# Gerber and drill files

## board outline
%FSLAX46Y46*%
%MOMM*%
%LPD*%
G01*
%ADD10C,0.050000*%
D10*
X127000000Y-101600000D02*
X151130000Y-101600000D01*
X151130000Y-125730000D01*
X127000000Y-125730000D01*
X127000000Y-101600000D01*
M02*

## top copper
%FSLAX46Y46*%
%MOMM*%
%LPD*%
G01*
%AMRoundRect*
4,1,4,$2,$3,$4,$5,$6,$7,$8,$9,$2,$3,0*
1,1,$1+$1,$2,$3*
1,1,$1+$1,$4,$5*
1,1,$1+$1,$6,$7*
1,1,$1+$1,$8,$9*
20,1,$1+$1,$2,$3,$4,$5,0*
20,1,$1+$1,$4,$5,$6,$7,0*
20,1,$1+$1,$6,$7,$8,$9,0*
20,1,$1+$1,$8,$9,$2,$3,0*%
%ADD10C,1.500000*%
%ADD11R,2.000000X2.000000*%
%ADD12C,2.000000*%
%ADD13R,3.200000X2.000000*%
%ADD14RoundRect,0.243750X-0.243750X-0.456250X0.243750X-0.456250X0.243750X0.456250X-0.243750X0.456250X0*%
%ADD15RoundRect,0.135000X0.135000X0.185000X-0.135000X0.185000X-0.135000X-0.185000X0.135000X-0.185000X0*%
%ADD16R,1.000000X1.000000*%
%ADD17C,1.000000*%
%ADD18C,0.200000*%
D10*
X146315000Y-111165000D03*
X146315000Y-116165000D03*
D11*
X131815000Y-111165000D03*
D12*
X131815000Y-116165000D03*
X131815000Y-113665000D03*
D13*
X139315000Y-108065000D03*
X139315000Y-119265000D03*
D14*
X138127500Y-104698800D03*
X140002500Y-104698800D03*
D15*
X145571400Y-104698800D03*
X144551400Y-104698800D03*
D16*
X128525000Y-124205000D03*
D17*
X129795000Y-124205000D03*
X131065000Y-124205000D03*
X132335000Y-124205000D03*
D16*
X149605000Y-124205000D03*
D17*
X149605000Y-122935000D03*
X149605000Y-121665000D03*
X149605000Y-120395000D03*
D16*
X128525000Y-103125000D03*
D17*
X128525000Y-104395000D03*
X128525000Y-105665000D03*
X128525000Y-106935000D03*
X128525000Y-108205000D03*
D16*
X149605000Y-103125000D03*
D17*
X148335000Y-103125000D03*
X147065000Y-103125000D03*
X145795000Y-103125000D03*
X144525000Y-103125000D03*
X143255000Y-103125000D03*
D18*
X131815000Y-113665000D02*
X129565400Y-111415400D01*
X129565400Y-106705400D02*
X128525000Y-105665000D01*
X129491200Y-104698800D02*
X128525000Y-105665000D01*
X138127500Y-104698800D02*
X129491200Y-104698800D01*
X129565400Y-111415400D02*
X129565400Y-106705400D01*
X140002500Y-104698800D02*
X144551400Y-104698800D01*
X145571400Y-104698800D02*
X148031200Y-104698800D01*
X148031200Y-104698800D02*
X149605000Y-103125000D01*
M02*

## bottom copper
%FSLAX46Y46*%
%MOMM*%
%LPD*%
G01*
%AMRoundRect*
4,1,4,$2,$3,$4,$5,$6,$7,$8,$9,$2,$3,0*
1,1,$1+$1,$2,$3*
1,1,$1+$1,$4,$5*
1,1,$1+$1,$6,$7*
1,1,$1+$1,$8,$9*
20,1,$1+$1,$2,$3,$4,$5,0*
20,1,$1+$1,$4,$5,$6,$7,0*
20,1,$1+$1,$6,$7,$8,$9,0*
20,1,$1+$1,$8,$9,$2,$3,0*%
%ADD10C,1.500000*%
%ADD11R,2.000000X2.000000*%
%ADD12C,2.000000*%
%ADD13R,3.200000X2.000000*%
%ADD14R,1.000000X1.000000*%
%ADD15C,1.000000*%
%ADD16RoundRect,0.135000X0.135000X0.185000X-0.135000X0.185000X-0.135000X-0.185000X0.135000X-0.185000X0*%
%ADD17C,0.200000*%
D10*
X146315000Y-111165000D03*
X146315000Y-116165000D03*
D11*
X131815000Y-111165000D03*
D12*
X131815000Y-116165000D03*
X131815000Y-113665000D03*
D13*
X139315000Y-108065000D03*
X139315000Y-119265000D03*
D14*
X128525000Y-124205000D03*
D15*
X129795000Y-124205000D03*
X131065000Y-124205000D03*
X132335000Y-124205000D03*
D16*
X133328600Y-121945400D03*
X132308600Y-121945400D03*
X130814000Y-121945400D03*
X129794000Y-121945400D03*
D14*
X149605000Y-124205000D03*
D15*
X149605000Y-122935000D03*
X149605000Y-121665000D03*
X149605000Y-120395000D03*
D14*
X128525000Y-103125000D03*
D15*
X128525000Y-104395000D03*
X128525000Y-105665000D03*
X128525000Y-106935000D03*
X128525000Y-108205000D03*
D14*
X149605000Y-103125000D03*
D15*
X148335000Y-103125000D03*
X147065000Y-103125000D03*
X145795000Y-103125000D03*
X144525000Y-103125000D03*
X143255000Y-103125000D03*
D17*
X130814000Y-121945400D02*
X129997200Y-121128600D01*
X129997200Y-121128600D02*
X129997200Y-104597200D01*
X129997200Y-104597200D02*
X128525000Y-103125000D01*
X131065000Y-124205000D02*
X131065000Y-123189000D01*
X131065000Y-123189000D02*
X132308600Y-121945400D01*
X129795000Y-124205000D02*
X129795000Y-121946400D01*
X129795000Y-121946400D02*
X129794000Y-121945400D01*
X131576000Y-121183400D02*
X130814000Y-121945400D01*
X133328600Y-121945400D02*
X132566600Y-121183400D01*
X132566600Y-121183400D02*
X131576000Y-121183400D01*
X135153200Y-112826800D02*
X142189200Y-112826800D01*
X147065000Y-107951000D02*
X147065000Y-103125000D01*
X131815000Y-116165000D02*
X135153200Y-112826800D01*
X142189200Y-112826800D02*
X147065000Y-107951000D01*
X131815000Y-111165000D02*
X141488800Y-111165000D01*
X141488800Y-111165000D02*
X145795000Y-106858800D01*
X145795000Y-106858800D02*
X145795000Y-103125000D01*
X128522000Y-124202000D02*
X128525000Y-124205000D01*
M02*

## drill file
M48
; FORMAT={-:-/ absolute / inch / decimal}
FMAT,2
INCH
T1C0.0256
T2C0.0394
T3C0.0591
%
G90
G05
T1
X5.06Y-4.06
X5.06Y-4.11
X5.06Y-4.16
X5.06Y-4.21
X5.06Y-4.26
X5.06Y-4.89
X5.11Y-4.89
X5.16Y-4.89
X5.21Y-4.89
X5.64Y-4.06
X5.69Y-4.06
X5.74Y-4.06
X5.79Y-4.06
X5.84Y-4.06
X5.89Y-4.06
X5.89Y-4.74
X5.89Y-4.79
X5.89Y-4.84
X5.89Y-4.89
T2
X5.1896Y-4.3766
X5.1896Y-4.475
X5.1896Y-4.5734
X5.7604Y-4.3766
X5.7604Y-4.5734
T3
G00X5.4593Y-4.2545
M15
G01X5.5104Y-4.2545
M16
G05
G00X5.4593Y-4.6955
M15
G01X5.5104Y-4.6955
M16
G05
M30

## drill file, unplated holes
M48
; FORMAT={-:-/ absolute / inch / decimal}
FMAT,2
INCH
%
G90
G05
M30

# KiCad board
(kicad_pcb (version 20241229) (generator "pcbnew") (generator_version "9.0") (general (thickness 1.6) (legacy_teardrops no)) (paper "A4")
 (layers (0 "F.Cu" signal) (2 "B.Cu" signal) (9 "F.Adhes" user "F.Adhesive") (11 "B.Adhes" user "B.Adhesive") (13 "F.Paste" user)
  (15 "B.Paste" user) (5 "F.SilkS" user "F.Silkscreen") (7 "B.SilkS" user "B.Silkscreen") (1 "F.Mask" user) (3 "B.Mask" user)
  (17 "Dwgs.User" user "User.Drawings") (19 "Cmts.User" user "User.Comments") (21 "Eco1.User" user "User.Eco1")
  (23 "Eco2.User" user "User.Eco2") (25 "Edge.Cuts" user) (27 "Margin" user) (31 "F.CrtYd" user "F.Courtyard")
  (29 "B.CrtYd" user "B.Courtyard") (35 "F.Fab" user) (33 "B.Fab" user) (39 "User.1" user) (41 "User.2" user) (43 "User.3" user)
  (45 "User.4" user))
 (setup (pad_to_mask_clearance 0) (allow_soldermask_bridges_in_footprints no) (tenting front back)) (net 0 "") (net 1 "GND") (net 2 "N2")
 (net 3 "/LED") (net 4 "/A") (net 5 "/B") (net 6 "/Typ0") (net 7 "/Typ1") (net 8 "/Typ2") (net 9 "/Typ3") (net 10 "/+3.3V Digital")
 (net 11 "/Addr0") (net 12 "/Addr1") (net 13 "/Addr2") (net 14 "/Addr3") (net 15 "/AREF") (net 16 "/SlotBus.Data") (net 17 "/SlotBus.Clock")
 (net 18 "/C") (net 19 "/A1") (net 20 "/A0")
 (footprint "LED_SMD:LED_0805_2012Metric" (layer "F.Cu") (at 139.065 104.6988)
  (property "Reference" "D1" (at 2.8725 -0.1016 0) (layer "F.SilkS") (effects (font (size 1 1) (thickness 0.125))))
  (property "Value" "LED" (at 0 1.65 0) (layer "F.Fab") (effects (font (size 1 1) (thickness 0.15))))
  (pad "1" smd roundrect (at -0.9375 0) (size 0.975 1.4) (layers "F.Cu" "F.Mask" "F.Paste") (roundrect_rratio 0.25) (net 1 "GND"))
  (pad "2" smd roundrect (at 0.9375 0) (size 0.975 1.4) (layers "F.Cu" "F.Mask" "F.Paste") (roundrect_rratio 0.25) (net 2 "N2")))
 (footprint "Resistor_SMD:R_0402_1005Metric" (layer "F.Cu") (at 145.0614 104.6988 180)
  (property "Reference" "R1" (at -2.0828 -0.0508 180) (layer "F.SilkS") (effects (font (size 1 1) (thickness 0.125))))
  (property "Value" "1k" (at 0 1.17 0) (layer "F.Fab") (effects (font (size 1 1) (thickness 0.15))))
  (pad "1" smd roundrect (at -0.51 0 180) (size 0.54 0.64) (layers "F.Cu" "F.Mask" "F.Paste") (roundrect_rratio 0.25) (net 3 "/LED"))
  (pad "2" smd roundrect (at 0.51 0 180) (size 0.54 0.64) (layers "F.Cu" "F.Mask" "F.Paste") (roundrect_rratio 0.25) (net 2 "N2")))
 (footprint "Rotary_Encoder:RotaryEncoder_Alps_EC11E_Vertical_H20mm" (layer "F.Cu") (at 131.815 111.165)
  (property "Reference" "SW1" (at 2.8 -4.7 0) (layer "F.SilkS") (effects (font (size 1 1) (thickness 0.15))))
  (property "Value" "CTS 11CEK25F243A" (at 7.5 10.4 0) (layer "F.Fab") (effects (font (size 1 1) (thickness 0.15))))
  (pad "" thru_hole circle (at 14.5 0) (size 1.5 1.5) (drill 1) (layers "*.Cu" "*.Mask") (remove_unused_layers no))
  (pad "" thru_hole circle (at 14.5 5) (size 1.5 1.5) (drill 1) (layers "*.Cu" "*.Mask") (remove_unused_layers no))
  (pad "A" thru_hole rect (at 0 0) (size 2 2) (drill 1) (layers "*.Cu" "*.Mask") (remove_unused_layers no) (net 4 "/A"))
  (pad "B" thru_hole circle (at 0 5) (size 2 2) (drill 1) (layers "*.Cu" "*.Mask") (remove_unused_layers no) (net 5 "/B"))
  (pad "C" thru_hole circle (at 0 2.5) (size 2 2) (drill 1) (layers "*.Cu" "*.Mask") (remove_unused_layers no) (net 1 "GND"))
  (pad "MP" thru_hole rect (at 7.5 -3.1) (size 3.2 2) (drill oval 2.8 1.5) (layers "*.Cu" "*.Mask") (remove_unused_layers no))
  (pad "MP" thru_hole rect (at 7.5 8.1) (size 3.2 2) (drill oval 2.8 1.5) (layers "*.Cu" "*.Mask") (remove_unused_layers no)))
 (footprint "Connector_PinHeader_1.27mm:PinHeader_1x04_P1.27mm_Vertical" (layer "B.Cu") (at 128.525 124.205 -90)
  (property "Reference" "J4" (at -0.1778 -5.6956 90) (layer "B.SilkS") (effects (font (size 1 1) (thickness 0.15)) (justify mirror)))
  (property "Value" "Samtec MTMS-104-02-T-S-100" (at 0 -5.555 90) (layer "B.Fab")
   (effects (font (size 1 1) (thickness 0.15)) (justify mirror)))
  (pad "1" thru_hole rect (at 0 0 270) (size 1 1) (drill 0.65) (layers "*.Cu" "*.Mask") (remove_unused_layers no) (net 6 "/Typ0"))
  (pad "2" thru_hole circle (at 0 -1.27 270) (size 1 1) (drill 0.65) (layers "*.Cu" "*.Mask") (remove_unused_layers no) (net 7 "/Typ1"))
  (pad "3" thru_hole circle (at 0 -2.54 270) (size 1 1) (drill 0.65) (layers "*.Cu" "*.Mask") (remove_unused_layers no) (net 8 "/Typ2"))
  (pad "4" thru_hole circle (at 0 -3.81 270) (size 1 1) (drill 0.65) (layers "*.Cu" "*.Mask") (remove_unused_layers no) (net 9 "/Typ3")))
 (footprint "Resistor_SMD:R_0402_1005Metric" (layer "B.Cu") (at 132.8186 121.9454 180)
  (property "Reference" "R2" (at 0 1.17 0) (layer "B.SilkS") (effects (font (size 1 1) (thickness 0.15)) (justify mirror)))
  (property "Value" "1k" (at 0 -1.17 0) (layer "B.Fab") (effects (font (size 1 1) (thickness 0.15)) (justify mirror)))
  (pad "1" smd roundrect (at -0.51 0 180) (size 0.54 0.64) (layers "B.Cu" "B.Mask" "B.Paste") (roundrect_rratio 0.25)
   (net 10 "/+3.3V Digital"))
  (pad "2" smd roundrect (at 0.51 0 180) (size 0.54 0.64) (layers "B.Cu" "B.Mask" "B.Paste") (roundrect_rratio 0.25) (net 8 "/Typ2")))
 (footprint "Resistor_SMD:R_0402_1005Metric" (layer "B.Cu") (at 130.304 121.9454 180)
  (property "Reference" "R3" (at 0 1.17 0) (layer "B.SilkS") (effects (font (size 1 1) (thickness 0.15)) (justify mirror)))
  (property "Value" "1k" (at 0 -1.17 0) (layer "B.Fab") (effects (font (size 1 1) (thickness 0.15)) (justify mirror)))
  (pad "1" smd roundrect (at -0.51 0 180) (size 0.54 0.64) (layers "B.Cu" "B.Mask" "B.Paste") (roundrect_rratio 0.25)
   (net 10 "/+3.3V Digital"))
  (pad "2" smd roundrect (at 0.51 0 180) (size 0.54 0.64) (layers "B.Cu" "B.Mask" "B.Paste") (roundrect_rratio 0.25) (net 7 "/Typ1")))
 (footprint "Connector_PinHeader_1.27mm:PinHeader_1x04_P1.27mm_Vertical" (layer "B.Cu") (at 149.605 124.205)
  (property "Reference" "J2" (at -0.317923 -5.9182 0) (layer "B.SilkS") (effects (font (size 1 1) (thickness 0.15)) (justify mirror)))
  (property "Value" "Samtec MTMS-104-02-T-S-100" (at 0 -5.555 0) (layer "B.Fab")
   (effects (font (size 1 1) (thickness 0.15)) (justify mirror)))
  (pad "1" thru_hole rect (at 0 0) (size 1 1) (drill 0.65) (layers "*.Cu" "*.Mask") (remove_unused_layers no) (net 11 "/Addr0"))
  (pad "2" thru_hole circle (at 0 -1.27) (size 1 1) (drill 0.65) (layers "*.Cu" "*.Mask") (remove_unused_layers no) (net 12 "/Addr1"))
  (pad "3" thru_hole circle (at 0 -2.54) (size 1 1) (drill 0.65) (layers "*.Cu" "*.Mask") (remove_unused_layers no) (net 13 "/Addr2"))
  (pad "4" thru_hole circle (at 0 -3.81) (size 1 1) (drill 0.65) (layers "*.Cu" "*.Mask") (remove_unused_layers no) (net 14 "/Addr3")))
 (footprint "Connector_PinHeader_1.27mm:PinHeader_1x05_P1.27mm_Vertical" (layer "B.Cu") (at 128.525 103.125 180)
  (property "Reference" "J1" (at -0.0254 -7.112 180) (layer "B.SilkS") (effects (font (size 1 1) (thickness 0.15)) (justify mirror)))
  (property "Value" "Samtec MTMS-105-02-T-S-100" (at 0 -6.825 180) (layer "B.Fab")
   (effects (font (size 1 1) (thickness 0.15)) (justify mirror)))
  (pad "1" thru_hole rect (at 0 0 180) (size 1 1) (drill 0.65) (layers "*.Cu" "*.Mask") (remove_unused_layers no) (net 10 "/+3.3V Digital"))
  (pad "2" thru_hole circle (at 0 -1.27 180) (size 1 1) (drill 0.65) (layers "*.Cu" "*.Mask") (remove_unused_layers no) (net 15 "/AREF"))
  (pad "3" thru_hole circle (at 0 -2.54 180) (size 1 1) (drill 0.65) (layers "*.Cu" "*.Mask") (remove_unused_layers no) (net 1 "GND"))
  (pad "4" thru_hole circle (at 0 -3.81 180) (size 1 1) (drill 0.65) (layers "*.Cu" "*.Mask") (remove_unused_layers no)
   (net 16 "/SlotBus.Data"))
  (pad "5" thru_hole circle (at 0 -5.08 180) (size 1 1) (drill 0.65) (layers "*.Cu" "*.Mask") (remove_unused_layers no)
   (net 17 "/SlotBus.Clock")))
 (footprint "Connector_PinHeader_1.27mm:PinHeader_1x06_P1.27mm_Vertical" (layer "B.Cu") (at 149.605 103.125 90)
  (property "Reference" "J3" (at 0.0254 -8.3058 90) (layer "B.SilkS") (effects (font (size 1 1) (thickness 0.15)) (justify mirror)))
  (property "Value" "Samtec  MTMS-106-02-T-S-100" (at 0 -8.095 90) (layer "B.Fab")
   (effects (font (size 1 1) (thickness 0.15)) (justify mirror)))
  (pad "1" thru_hole rect (at 0 0 90) (size 1 1) (drill 0.65) (layers "*.Cu" "*.Mask") (remove_unused_layers no) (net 3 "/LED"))
  (pad "2" thru_hole circle (at 0 -1.27 90) (size 1 1) (drill 0.65) (layers "*.Cu" "*.Mask") (remove_unused_layers no) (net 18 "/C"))
  (pad "3" thru_hole circle (at 0 -2.54 90) (size 1 1) (drill 0.65) (layers "*.Cu" "*.Mask") (remove_unused_layers no) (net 5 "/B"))
  (pad "4" thru_hole circle (at 0 -3.81 90) (size 1 1) (drill 0.65) (layers "*.Cu" "*.Mask") (remove_unused_layers no) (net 4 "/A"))
  (pad "5" thru_hole circle (at 0 -5.08 90) (size 1 1) (drill 0.65) (layers "*.Cu" "*.Mask") (remove_unused_layers no) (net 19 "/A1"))
  (pad "6" thru_hole circle (at 0 -6.35 90) (size 1 1) (drill 0.65) (layers "*.Cu" "*.Mask") (remove_unused_layers no) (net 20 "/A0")))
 (gr_rect (start 127 101.6) (end 151.13 125.73) (stroke (width 0.05) (type solid)) (fill no) (layer "Edge.Cuts"))
 (segment (start 131.815 113.665) (end 129.5654 111.4154) (width 0.2) (layer "F.Cu") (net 1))
 (segment (start 129.5654 106.7054) (end 128.525 105.665) (width 0.2) (layer "F.Cu") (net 1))
 (segment (start 129.4912 104.6988) (end 128.525 105.665) (width 0.2) (layer "F.Cu") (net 1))
 (segment (start 138.1275 104.6988) (end 129.4912 104.6988) (width 0.2) (layer "F.Cu") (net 1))
 (segment (start 129.5654 111.4154) (end 129.5654 106.7054) (width 0.2) (layer "F.Cu") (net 1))
 (segment (start 140.0025 104.6988) (end 144.5514 104.6988) (width 0.2) (layer "F.Cu") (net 2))
 (segment (start 131.576 121.1834) (end 130.814 121.9454) (width 0.2) (layer "B.Cu") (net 10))
 (segment (start 133.3286 121.9454) (end 132.5666 121.1834) (width 0.2) (layer "B.Cu") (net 10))
 (segment (start 129.9972 121.1286) (end 129.9972 104.5972) (width 0.2) (layer "B.Cu") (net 10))
 (segment (start 129.9972 104.5972) (end 128.525 103.125) (width 0.2) (layer "B.Cu") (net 10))
 (segment (start 130.814 121.9454) (end 129.9972 121.1286) (width 0.2) (layer "B.Cu") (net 10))
 (segment (start 132.5666 121.1834) (end 131.576 121.1834) (width 0.2) (layer "B.Cu") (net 10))
 (segment (start 135.1532 112.8268) (end 142.1892 112.8268) (width 0.2) (layer "B.Cu") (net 5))
 (segment (start 147.065 107.951) (end 147.065 103.125) (width 0.2) (layer "B.Cu") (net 5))
 (segment (start 131.815 116.165) (end 135.1532 112.8268) (width 0.2) (layer "B.Cu") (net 5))
 (segment (start 142.1892 112.8268) (end 147.065 107.951) (width 0.2) (layer "B.Cu") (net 5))
 (segment (start 145.5714 104.6988) (end 148.0312 104.6988) (width 0.2) (layer "F.Cu") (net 3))
 (segment (start 148.0312 104.6988) (end 149.605 103.125) (width 0.2) (layer "F.Cu") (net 3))
 (segment (start 131.815 111.165) (end 141.4888 111.165) (width 0.2) (layer "B.Cu") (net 4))
 (segment (start 141.4888 111.165) (end 145.795 106.8588) (width 0.2) (layer "B.Cu") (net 4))
 (segment (start 145.795 106.8588) (end 145.795 103.125) (width 0.2) (layer "B.Cu") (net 4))
 (segment (start 128.522 124.202) (end 128.525 124.205) (width 0.2) (layer "B.Cu") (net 6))
 (segment (start 129.795 121.9464) (end 129.794 121.9454) (width 0.2) (layer "B.Cu") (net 7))
 (segment (start 129.795 124.205) (end 129.795 121.9464) (width 0.2) (layer "B.Cu") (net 7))
 (segment (start 131.065 123.189) (end 132.3086 121.9454) (width 0.2) (layer "B.Cu") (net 8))
 (segment (start 131.065 124.205) (end 131.065 123.189) (width 0.2) (layer "B.Cu") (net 8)))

